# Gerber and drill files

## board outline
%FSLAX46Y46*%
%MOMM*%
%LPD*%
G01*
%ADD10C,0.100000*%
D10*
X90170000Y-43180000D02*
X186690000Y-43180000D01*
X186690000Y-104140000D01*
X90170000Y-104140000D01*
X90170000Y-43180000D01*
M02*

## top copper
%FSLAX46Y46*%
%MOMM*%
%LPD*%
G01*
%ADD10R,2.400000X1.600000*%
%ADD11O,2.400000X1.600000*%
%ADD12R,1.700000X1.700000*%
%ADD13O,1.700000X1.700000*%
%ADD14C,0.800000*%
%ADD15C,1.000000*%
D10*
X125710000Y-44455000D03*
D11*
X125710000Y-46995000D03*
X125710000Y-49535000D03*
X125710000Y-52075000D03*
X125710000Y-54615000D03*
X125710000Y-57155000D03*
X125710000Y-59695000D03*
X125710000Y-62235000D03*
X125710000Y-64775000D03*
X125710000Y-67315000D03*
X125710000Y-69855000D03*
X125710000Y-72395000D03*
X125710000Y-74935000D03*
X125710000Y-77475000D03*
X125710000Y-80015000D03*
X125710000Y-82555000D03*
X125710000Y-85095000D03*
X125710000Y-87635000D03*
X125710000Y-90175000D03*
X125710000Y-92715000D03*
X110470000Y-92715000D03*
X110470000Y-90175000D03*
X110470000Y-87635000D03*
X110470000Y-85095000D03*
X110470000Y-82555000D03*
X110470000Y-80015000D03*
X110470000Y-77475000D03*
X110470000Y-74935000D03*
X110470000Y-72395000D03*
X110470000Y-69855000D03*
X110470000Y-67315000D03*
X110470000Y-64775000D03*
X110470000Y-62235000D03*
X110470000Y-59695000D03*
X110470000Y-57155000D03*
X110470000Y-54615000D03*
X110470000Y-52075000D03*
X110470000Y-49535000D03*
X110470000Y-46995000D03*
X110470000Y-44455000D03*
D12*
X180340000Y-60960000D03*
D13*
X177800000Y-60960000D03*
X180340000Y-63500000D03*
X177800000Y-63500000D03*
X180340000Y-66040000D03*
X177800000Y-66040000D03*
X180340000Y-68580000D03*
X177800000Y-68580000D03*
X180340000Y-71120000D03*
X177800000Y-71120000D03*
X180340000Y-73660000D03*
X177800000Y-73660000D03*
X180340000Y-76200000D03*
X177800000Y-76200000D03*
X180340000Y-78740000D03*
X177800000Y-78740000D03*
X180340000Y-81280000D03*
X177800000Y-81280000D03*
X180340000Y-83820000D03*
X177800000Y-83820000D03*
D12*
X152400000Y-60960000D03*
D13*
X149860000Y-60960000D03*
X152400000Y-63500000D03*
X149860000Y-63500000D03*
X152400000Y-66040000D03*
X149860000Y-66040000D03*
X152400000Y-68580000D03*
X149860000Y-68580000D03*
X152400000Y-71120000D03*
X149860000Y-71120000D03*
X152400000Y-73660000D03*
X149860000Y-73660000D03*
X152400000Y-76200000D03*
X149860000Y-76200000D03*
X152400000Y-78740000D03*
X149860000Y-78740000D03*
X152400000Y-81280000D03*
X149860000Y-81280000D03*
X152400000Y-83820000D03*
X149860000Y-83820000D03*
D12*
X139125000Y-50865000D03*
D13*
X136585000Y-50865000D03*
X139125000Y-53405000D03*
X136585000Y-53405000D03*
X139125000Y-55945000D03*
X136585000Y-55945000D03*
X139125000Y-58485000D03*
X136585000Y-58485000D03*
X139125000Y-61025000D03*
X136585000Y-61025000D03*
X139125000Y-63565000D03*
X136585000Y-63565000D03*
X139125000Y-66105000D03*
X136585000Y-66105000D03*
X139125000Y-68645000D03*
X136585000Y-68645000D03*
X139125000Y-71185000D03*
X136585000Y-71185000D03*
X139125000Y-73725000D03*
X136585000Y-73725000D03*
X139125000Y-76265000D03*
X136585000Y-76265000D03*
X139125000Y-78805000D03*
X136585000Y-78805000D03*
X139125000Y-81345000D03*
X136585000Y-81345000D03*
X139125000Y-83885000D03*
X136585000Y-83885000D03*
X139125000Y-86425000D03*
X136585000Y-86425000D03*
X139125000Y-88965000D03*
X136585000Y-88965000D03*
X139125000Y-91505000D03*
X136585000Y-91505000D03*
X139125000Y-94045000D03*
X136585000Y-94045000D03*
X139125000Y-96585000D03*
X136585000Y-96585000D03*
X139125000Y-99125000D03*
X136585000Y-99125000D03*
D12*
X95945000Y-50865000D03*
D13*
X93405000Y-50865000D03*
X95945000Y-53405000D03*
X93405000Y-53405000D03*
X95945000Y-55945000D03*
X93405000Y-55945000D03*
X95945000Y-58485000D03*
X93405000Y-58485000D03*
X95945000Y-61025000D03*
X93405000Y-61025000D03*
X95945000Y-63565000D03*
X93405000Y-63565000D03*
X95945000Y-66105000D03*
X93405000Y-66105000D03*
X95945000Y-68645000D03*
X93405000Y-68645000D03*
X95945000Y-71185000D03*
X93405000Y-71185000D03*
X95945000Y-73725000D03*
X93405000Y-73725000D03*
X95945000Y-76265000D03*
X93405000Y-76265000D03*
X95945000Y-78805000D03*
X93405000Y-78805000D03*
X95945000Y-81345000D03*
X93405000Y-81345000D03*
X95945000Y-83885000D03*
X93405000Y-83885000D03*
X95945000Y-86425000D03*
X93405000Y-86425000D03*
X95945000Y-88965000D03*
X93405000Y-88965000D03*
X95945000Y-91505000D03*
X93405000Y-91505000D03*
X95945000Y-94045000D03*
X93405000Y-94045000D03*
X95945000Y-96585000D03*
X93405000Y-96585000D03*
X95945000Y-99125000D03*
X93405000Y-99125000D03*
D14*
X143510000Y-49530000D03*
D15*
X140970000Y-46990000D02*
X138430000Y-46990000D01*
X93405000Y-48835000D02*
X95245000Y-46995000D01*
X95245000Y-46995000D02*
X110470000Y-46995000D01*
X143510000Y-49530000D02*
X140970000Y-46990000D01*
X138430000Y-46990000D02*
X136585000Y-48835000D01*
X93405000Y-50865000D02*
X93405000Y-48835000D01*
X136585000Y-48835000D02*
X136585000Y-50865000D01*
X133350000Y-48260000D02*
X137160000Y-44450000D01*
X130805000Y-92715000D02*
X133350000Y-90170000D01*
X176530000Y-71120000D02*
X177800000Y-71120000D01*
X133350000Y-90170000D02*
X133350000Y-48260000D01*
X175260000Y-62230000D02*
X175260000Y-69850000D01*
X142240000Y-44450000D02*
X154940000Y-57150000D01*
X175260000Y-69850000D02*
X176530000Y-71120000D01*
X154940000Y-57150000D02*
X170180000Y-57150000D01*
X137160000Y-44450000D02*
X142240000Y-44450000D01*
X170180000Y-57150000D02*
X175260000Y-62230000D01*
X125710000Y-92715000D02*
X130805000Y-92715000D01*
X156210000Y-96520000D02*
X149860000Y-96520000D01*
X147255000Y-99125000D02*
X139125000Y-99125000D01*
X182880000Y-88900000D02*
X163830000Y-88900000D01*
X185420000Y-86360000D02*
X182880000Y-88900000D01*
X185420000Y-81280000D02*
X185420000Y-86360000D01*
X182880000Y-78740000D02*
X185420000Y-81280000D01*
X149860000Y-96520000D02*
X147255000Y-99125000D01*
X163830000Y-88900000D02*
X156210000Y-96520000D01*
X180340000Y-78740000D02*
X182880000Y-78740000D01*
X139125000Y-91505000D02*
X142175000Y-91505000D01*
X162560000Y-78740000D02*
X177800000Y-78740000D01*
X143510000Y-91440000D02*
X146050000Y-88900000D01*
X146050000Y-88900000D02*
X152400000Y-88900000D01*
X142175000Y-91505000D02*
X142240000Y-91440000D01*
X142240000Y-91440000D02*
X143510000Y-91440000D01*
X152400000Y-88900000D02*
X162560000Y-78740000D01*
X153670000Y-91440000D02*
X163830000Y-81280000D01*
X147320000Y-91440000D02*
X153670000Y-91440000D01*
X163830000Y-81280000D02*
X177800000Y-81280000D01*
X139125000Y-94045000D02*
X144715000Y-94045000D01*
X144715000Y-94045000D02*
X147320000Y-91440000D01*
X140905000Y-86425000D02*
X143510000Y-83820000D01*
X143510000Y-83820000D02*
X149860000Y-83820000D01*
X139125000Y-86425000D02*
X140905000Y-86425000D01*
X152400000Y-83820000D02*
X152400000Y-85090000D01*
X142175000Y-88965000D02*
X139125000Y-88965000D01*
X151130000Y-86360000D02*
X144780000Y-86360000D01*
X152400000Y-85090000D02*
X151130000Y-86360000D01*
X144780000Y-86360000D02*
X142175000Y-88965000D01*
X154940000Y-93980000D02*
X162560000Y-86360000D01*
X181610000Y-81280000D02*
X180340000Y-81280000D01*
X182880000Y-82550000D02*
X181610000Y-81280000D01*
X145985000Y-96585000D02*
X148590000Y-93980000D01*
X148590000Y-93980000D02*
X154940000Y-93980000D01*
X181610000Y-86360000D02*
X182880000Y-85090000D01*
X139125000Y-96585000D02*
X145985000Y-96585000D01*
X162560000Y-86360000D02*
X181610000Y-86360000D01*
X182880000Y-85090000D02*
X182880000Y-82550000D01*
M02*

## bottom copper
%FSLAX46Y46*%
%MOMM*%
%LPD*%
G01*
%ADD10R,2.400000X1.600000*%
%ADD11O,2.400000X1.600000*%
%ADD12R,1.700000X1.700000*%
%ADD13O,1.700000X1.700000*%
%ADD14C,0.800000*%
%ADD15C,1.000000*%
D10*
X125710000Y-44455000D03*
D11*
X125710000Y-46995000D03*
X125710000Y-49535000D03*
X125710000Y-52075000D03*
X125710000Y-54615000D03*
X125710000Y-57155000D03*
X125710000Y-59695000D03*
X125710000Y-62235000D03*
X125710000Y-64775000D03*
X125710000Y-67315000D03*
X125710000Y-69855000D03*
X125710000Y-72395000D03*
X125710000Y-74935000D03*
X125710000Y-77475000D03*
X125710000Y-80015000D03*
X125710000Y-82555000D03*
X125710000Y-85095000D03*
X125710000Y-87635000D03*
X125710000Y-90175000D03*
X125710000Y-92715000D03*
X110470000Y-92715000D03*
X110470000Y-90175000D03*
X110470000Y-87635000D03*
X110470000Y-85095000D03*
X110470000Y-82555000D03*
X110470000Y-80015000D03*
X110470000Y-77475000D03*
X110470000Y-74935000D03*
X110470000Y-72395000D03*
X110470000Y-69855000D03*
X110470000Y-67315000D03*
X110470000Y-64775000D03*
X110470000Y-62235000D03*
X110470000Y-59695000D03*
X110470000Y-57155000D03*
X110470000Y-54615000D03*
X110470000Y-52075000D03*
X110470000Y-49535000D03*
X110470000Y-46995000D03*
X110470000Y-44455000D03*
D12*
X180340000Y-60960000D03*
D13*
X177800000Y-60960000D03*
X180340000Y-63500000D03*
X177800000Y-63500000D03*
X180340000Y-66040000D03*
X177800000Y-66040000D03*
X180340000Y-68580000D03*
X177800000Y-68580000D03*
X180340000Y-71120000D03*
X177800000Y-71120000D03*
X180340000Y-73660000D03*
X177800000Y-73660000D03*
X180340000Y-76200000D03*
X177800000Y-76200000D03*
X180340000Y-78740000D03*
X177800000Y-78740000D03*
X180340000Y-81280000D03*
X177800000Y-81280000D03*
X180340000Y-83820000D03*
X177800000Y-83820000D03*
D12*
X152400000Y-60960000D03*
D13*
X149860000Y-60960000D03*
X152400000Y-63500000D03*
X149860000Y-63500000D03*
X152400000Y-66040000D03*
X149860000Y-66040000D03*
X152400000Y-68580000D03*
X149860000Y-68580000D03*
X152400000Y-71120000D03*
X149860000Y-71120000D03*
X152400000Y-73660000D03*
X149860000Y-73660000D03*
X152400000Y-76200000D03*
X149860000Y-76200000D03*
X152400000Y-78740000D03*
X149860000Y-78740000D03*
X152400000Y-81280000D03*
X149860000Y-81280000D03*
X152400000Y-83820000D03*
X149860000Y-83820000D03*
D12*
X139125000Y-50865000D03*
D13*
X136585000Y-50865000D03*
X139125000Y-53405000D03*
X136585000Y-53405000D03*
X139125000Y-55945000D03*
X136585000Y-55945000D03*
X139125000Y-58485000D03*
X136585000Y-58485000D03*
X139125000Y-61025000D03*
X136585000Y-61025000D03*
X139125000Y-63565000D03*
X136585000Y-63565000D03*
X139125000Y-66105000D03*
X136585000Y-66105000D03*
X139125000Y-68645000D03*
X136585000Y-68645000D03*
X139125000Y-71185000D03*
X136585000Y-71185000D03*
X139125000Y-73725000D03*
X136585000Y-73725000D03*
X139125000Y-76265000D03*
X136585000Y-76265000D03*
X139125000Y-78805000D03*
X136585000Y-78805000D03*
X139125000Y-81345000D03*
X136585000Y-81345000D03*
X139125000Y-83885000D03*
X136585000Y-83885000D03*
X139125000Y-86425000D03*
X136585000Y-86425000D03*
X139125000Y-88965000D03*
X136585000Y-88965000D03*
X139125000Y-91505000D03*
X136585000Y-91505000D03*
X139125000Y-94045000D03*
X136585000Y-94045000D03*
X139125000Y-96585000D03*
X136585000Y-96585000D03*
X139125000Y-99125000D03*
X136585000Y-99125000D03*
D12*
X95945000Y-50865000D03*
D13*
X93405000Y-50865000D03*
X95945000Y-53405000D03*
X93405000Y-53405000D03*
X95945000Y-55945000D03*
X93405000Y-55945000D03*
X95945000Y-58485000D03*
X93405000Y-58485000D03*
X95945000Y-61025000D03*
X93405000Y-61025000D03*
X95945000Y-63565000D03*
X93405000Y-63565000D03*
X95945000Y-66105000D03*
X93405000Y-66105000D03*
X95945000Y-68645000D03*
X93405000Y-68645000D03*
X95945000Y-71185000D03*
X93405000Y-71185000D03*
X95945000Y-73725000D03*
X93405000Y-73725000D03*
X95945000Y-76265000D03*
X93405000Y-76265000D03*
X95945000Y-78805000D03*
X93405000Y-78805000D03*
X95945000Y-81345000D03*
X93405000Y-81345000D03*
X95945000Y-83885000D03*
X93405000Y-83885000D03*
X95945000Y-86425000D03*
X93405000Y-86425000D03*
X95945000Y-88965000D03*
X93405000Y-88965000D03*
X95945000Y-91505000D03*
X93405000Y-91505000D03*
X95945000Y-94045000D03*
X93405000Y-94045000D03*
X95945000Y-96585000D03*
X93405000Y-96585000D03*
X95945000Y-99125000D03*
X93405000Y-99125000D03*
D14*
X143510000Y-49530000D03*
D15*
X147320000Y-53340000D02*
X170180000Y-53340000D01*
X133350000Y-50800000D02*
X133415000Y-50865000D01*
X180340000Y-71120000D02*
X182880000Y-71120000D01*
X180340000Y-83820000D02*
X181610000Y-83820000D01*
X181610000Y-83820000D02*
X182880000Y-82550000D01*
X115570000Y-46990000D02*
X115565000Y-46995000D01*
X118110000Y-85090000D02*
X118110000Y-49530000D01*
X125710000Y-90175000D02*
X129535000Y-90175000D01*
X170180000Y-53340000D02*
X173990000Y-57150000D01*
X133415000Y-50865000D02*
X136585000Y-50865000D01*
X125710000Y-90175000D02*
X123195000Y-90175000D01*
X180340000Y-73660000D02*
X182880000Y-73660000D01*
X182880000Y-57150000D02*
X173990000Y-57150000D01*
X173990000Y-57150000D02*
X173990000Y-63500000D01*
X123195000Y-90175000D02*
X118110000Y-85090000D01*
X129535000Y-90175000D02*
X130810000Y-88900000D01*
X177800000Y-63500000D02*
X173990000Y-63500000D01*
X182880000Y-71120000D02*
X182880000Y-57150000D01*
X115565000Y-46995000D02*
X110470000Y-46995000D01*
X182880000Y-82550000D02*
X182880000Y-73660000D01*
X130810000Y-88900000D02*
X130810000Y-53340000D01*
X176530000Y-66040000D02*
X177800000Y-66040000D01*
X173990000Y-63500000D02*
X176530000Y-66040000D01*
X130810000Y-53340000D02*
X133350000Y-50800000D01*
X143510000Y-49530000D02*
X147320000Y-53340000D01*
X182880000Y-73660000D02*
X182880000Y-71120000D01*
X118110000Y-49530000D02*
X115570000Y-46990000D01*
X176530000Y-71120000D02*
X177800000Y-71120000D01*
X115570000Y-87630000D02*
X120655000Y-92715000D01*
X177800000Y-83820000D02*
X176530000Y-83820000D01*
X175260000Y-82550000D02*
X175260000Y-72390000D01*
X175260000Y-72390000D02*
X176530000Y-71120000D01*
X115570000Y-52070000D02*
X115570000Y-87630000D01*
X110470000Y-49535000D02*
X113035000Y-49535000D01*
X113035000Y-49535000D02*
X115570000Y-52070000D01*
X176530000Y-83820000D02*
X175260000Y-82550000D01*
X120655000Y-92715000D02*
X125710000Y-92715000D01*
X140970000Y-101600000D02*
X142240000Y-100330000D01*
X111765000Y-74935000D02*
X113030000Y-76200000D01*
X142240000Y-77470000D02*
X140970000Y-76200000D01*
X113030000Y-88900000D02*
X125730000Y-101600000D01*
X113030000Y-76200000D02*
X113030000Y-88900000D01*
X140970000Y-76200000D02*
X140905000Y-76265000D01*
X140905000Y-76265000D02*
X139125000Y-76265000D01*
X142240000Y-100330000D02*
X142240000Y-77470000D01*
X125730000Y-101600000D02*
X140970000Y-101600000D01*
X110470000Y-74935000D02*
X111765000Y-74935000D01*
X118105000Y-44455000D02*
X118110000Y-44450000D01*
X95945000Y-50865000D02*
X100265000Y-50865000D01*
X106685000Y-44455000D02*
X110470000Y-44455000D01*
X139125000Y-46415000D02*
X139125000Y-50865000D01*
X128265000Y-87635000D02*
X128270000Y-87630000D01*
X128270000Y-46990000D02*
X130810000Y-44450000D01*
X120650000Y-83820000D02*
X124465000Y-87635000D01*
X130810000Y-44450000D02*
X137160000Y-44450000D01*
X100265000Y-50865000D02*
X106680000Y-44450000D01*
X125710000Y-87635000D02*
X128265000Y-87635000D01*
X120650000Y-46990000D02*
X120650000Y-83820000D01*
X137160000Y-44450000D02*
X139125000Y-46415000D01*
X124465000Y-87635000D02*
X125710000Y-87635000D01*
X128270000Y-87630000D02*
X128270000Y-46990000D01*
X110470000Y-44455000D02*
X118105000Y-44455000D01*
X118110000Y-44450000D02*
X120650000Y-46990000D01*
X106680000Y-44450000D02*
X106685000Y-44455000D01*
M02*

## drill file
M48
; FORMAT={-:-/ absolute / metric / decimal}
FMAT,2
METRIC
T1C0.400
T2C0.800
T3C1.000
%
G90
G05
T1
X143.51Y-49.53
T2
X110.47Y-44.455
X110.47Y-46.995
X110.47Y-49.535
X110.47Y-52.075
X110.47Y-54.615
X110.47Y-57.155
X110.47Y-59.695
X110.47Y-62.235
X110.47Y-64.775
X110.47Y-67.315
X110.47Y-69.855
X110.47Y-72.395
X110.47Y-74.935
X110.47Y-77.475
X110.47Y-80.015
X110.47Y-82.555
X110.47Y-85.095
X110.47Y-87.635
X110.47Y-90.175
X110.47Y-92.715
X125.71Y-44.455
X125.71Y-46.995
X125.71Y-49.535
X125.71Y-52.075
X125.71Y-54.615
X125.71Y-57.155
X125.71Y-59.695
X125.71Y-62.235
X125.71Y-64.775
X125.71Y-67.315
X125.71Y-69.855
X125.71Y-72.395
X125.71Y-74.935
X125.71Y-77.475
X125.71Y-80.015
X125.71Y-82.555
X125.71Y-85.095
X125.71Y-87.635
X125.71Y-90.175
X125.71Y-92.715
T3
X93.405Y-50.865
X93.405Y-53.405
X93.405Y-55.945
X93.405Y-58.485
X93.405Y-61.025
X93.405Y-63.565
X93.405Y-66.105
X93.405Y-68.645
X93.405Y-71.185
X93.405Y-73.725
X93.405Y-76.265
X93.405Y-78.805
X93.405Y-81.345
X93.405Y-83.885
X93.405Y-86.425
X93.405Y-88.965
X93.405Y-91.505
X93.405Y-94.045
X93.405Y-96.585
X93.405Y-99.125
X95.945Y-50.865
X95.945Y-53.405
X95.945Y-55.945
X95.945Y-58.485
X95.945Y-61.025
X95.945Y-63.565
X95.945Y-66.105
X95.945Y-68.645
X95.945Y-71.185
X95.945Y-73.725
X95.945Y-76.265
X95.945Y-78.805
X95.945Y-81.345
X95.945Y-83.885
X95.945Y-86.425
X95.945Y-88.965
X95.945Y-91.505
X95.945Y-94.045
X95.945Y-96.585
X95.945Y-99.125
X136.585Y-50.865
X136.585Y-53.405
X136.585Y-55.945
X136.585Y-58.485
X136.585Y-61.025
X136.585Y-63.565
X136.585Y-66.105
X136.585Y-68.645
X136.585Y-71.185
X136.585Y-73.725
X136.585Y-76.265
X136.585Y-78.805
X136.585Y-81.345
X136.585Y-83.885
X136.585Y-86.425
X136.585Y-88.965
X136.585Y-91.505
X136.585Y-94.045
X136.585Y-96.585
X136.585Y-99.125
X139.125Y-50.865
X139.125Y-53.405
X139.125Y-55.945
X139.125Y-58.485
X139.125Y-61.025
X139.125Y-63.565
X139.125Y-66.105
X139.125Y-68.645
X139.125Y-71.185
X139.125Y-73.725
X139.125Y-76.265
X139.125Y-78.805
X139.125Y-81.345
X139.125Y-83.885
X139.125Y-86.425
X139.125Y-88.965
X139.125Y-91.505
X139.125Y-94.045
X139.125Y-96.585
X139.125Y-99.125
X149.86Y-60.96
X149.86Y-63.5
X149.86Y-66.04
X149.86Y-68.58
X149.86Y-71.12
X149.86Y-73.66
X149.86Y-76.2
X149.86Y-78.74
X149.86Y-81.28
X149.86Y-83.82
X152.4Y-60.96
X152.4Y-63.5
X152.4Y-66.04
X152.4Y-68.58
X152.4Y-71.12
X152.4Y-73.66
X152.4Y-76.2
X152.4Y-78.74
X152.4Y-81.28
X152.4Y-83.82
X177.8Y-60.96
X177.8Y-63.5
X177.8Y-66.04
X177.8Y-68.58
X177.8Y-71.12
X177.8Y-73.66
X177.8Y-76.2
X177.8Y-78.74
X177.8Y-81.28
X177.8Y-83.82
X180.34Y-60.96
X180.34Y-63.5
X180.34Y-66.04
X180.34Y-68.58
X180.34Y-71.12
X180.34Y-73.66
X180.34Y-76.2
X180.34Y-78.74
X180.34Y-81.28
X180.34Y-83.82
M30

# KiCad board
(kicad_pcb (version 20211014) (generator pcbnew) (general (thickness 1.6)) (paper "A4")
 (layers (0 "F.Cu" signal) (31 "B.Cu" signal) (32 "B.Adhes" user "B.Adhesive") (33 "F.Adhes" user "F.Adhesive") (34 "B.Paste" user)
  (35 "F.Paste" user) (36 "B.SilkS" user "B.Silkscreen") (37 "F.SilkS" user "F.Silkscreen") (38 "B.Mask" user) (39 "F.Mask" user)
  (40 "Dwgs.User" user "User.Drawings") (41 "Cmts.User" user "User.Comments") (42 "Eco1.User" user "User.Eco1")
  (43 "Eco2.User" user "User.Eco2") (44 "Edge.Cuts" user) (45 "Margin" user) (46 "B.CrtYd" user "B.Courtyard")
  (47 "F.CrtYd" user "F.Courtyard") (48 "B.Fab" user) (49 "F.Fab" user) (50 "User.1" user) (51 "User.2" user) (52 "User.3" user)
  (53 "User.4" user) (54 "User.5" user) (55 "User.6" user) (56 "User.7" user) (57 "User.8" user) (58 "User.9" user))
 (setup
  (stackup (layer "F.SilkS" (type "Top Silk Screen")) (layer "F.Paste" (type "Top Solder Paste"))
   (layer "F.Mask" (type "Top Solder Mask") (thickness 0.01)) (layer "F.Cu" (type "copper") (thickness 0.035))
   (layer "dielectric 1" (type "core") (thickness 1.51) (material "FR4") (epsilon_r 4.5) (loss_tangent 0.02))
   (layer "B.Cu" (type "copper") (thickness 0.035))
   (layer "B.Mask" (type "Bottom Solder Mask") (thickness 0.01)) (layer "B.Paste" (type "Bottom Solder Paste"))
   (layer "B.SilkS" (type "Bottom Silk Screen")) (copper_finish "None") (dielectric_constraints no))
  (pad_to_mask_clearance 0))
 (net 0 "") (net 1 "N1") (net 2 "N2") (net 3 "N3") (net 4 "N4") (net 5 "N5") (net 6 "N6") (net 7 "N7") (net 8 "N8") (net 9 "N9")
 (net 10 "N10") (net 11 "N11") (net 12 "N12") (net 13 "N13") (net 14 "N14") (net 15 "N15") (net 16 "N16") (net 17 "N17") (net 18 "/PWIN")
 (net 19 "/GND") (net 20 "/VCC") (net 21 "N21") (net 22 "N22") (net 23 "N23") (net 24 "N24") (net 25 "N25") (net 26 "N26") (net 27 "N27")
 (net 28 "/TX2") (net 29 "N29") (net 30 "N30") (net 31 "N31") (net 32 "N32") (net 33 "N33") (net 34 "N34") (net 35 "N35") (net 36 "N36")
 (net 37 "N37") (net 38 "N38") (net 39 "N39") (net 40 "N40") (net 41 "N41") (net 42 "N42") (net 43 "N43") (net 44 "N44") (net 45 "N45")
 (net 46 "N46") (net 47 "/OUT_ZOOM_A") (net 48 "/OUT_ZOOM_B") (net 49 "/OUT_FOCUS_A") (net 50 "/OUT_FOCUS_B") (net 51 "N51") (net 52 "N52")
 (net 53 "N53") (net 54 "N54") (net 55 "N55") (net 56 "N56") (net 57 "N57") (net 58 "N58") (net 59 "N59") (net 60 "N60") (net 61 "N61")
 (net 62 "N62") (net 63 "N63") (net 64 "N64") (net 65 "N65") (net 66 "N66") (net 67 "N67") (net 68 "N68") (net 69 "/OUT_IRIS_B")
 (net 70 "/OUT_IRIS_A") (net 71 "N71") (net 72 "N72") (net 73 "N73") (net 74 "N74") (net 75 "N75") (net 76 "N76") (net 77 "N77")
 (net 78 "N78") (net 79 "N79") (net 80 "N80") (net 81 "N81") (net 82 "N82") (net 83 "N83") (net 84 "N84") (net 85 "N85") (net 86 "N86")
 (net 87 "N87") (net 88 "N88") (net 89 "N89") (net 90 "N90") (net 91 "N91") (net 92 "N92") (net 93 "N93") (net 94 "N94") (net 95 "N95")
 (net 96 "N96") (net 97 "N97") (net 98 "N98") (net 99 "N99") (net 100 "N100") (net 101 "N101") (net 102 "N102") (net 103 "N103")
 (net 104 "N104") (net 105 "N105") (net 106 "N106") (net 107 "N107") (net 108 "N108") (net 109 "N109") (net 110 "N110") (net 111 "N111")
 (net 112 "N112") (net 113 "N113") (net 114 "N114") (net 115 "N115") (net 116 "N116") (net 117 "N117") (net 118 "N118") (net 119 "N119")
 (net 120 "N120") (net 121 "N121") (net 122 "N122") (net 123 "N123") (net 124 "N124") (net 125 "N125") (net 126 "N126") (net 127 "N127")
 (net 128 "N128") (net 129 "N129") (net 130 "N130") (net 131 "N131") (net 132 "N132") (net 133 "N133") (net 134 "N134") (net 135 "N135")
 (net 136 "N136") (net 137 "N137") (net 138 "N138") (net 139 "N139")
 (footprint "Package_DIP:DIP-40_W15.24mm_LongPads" (layer "B.Cu") (at 125.71 44.455 180)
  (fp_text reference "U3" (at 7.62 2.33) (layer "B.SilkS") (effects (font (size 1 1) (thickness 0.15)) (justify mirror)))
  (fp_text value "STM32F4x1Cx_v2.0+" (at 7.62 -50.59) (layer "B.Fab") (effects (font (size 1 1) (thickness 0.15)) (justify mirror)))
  (pad "1" thru_hole rect locked (at 0 0 180) (size 2.4 1.6) (drill 0.8) (layers *.Cu *.Mask) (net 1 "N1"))
  (pad "2" thru_hole oval locked (at 0 -2.54 180) (size 2.4 1.6) (drill 0.8) (layers *.Cu *.Mask) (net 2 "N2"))
  (pad "3" thru_hole oval locked (at 0 -5.08 180) (size 2.4 1.6) (drill 0.8) (layers *.Cu *.Mask) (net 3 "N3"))
  (pad "4" thru_hole oval locked (at 0 -7.62 180) (size 2.4 1.6) (drill 0.8) (layers *.Cu *.Mask) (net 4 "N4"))
  (pad "5" thru_hole oval locked (at 0 -10.16 180) (size 2.4 1.6) (drill 0.8) (layers *.Cu *.Mask) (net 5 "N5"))
  (pad "6" thru_hole oval locked (at 0 -12.7 180) (size 2.4 1.6) (drill 0.8) (layers *.Cu *.Mask) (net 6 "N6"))
  (pad "7" thru_hole oval locked (at 0 -15.24 180) (size 2.4 1.6) (drill 0.8) (layers *.Cu *.Mask) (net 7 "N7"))
  (pad "8" thru_hole oval locked (at 0 -17.78 180) (size 2.4 1.6) (drill 0.8) (layers *.Cu *.Mask) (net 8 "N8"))
  (pad "9" thru_hole oval locked (at 0 -20.32 180) (size 2.4 1.6) (drill 0.8) (layers *.Cu *.Mask) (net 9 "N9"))
  (pad "10" thru_hole oval locked (at 0 -22.86 180) (size 2.4 1.6) (drill 0.8) (layers *.Cu *.Mask) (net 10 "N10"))
  (pad "11" thru_hole oval locked (at 0 -25.4 180) (size 2.4 1.6) (drill 0.8) (layers *.Cu *.Mask) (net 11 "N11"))
  (pad "12" thru_hole oval locked (at 0 -27.94 180) (size 2.4 1.6) (drill 0.8) (layers *.Cu *.Mask) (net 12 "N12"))
  (pad "13" thru_hole oval locked (at 0 -30.48 180) (size 2.4 1.6) (drill 0.8) (layers *.Cu *.Mask) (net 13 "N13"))
  (pad "14" thru_hole oval locked (at 0 -33.02 180) (size 2.4 1.6) (drill 0.8) (layers *.Cu *.Mask) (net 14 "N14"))
  (pad "15" thru_hole oval locked (at 0 -35.56 180) (size 2.4 1.6) (drill 0.8) (layers *.Cu *.Mask) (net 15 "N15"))
  (pad "16" thru_hole oval locked (at 0 -38.1 180) (size 2.4 1.6) (drill 0.8) (layers *.Cu *.Mask) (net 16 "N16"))
  (pad "17" thru_hole oval locked (at 0 -40.64 180) (size 2.4 1.6) (drill 0.8) (layers *.Cu *.Mask) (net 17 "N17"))
  (pad "18" thru_hole oval locked (at 0 -43.18 180) (size 2.4 1.6) (drill 0.8) (layers *.Cu *.Mask) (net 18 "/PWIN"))
  (pad "19" thru_hole oval locked (at 0 -45.72 180) (size 2.4 1.6) (drill 0.8) (layers *.Cu *.Mask) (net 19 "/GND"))
  (pad "20" thru_hole oval locked (at 0 -48.26 180) (size 2.4 1.6) (drill 0.8) (layers *.Cu *.Mask) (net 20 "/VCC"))
  (pad "21" thru_hole oval locked (at 15.24 -48.26 180) (size 2.4 1.6) (drill 0.8) (layers *.Cu *.Mask) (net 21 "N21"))
  (pad "22" thru_hole oval locked (at 15.24 -45.72 180) (size 2.4 1.6) (drill 0.8) (layers *.Cu *.Mask) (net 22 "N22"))
  (pad "23" thru_hole oval locked (at 15.24 -43.18 180) (size 2.4 1.6) (drill 0.8) (layers *.Cu *.Mask) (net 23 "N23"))
  (pad "24" thru_hole oval locked (at 15.24 -40.64 180) (size 2.4 1.6) (drill 0.8) (layers *.Cu *.Mask) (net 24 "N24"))
  (pad "25" thru_hole oval locked (at 15.24 -38.1 180) (size 2.4 1.6) (drill 0.8) (layers *.Cu *.Mask) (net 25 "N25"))
  (pad "26" thru_hole oval locked (at 15.24 -35.56 180) (size 2.4 1.6) (drill 0.8) (layers *.Cu *.Mask) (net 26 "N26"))
  (pad "27" thru_hole oval locked (at 15.24 -33.02 180) (size 2.4 1.6) (drill 0.8) (layers *.Cu *.Mask) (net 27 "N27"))
  (pad "28" thru_hole oval locked (at 15.24 -30.48 180) (size 2.4 1.6) (drill 0.8) (layers *.Cu *.Mask) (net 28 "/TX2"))
  (pad "29" thru_hole oval locked (at 15.24 -27.94 180) (size 2.4 1.6) (drill 0.8) (layers *.Cu *.Mask) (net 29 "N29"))
  (pad "30" thru_hole oval locked (at 15.24 -25.4 180) (size 2.4 1.6) (drill 0.8) (layers *.Cu *.Mask) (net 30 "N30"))
  (pad "31" thru_hole oval locked (at 15.24 -22.86 180) (size 2.4 1.6) (drill 0.8) (layers *.Cu *.Mask) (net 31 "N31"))
  (pad "32" thru_hole oval locked (at 15.24 -20.32 180) (size 2.4 1.6) (drill 0.8) (layers *.Cu *.Mask) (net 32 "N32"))
  (pad "33" thru_hole oval locked (at 15.24 -17.78 180) (size 2.4 1.6) (drill 0.8) (layers *.Cu *.Mask) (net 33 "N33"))
  (pad "34" thru_hole oval locked (at 15.24 -15.24 180) (size 2.4 1.6) (drill 0.8) (layers *.Cu *.Mask) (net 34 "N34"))
  (pad "35" thru_hole oval locked (at 15.24 -12.7 180) (size 2.4 1.6) (drill 0.8) (layers *.Cu *.Mask) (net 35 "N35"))
  (pad "36" thru_hole oval locked (at 15.24 -10.16 180) (size 2.4 1.6) (drill 0.8) (layers *.Cu *.Mask) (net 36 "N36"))
  (pad "37" thru_hole oval locked (at 15.24 -7.62 180) (size 2.4 1.6) (drill 0.8) (layers *.Cu *.Mask) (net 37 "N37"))
  (pad "38" thru_hole oval locked (at 15.24 -5.08 180) (size 2.4 1.6) (drill 0.8) (layers *.Cu *.Mask) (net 20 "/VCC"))
  (pad "39" thru_hole oval locked (at 15.24 -2.54 180) (size 2.4 1.6) (drill 0.8) (layers *.Cu *.Mask) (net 19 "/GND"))
  (pad "40" thru_hole oval locked (at 15.24 0 180) (size 2.4 1.6) (drill 0.8) (layers *.Cu *.Mask) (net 18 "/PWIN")))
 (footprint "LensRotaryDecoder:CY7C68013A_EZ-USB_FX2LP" (layer "B.Cu") (at 168.37 72.385 180)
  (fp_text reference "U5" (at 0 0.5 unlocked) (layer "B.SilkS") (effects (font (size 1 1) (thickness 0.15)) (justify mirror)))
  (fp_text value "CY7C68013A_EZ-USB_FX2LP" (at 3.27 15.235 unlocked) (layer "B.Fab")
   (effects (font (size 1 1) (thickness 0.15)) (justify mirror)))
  (pad "1" thru_hole rect (at -11.97 11.425 180) (size 1.7 1.7) (drill 1) (layers *.Cu *.Mask) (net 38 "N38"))
  (pad "2" thru_hole oval (at -9.43 11.425 180) (size 1.7 1.7) (drill 1) (layers *.Cu *.Mask) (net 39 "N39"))
  (pad "3" thru_hole oval (at -11.97 8.885 180) (size 1.7 1.7) (drill 1) (layers *.Cu *.Mask) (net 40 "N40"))
  (pad "4" thru_hole oval (at -9.43 8.885 180) (size 1.7 1.7) (drill 1) (layers *.Cu *.Mask) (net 19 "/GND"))
  (pad "5" thru_hole oval (at -11.97 6.345 180) (size 1.7 1.7) (drill 1) (layers *.Cu *.Mask) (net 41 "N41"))
  (pad "6" thru_hole oval (at -9.43 6.345 180) (size 1.7 1.7) (drill 1) (layers *.Cu *.Mask) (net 19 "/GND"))
  (pad "7" thru_hole oval (at -11.97 3.805 180) (size 1.7 1.7) (drill 1) (layers *.Cu *.Mask) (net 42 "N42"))
  (pad "8" thru_hole oval (at -9.43 3.805 180) (size 1.7 1.7) (drill 1) (layers *.Cu *.Mask) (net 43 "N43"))
  (pad "9" thru_hole oval (at -11.97 1.265 180) (size 1.7 1.7) (drill 1) (layers *.Cu *.Mask) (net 19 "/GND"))
  (pad "10" thru_hole oval (at -9.43 1.265 180) (size 1.7 1.7) (drill 1) (layers *.Cu *.Mask) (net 20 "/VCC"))
  (pad "11" thru_hole oval (at -11.97 -1.275 180) (size 1.7 1.7) (drill 1) (layers *.Cu *.Mask) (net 19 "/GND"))
  (pad "12" thru_hole oval (at -9.43 -1.275 180) (size 1.7 1.7) (drill 1) (layers *.Cu *.Mask) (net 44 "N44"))
  (pad "13" thru_hole oval (at -11.97 -3.815 180) (size 1.7 1.7) (drill 1) (layers *.Cu *.Mask) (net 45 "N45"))
  (pad "14" thru_hole oval (at -9.43 -3.815 180) (size 1.7 1.7) (drill 1) (layers *.Cu *.Mask) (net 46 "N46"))
  (pad "15" thru_hole oval (at -11.97 -6.355 180) (size 1.7 1.7) (drill 1) (layers *.Cu *.Mask) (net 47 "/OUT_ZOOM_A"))
  (pad "16" thru_hole oval (at -9.43 -6.355 180) (size 1.7 1.7) (drill 1) (layers *.Cu *.Mask) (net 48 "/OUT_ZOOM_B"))
  (pad "17" thru_hole oval (at -11.97 -8.895 180) (size 1.7 1.7) (drill 1) (layers *.Cu *.Mask) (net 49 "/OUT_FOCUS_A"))
  (pad "18" thru_hole oval (at -9.43 -8.895 180) (size 1.7 1.7) (drill 1) (layers *.Cu *.Mask) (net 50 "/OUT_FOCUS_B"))
  (pad "19" thru_hole oval (at -11.97 -11.435 180) (size 1.7 1.7) (drill 1) (layers *.Cu *.Mask) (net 19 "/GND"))
  (pad "20" thru_hole oval (at -9.43 -11.435 180) (size 1.7 1.7) (drill 1) (layers *.Cu *.Mask) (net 20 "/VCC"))
  (pad "21" thru_hole rect (at 15.97 11.425 180) (size 1.7 1.7) (drill 1) (layers *.Cu *.Mask) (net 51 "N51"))
  (pad "22" thru_hole oval (at 18.51 11.425 180) (size 1.7 1.7) (drill 1) (layers *.Cu *.Mask) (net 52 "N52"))
  (pad "23" thru_hole oval (at 15.97 8.885 180) (size 1.7 1.7) (drill 1) (layers *.Cu *.Mask) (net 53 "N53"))
  (pad "24" thru_hole oval (at 18.51 8.885 180) (size 1.7 1.7) (drill 1) (layers *.Cu *.Mask) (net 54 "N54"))
  (pad "25" thru_hole oval (at 15.97 6.345 180) (size 1.7 1.7) (drill 1) (layers *.Cu *.Mask) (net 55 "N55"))
  (pad "26" thru_hole oval (at 18.51 6.345 180) (size 1.7 1.7) (drill 1) (layers *.Cu *.Mask) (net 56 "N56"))
  (pad "27" thru_hole oval (at 15.97 3.805 180) (size 1.7 1.7) (drill 1) (layers *.Cu *.Mask) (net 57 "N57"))
  (pad "28" thru_hole oval (at 18.51 3.805 180) (size 1.7 1.7) (drill 1) (layers *.Cu *.Mask) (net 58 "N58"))
  (pad "29" thru_hole oval (at 15.97 1.265 180) (size 1.7 1.7) (drill 1) (layers *.Cu *.Mask) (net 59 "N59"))
  (pad "30" thru_hole oval (at 18.51 1.265 180) (size 1.7 1.7) (drill 1) (layers *.Cu *.Mask) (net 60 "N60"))
  (pad "31" thru_hole oval (at 15.97 -1.275 180) (size 1.7 1.7) (drill 1) (layers *.Cu *.Mask) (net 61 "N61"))
  (pad "32" thru_hole oval (at 18.51 -1.275 180) (size 1.7 1.7) (drill 1) (layers *.Cu *.Mask) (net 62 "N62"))
  (pad "33" thru_hole oval (at 15.97 -3.815 180) (size 1.7 1.7) (drill 1) (layers *.Cu *.Mask) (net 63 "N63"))
  (pad "34" thru_hole oval (at 18.51 -3.815 180) (size 1.7 1.7) (drill 1) (layers *.Cu *.Mask) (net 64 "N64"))
  (pad "35" thru_hole oval (at 15.97 -6.355 180) (size 1.7 1.7) (drill 1) (layers *.Cu *.Mask) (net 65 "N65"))
  (pad "36" thru_hole oval (at 18.51 -6.355 180) (size 1.7 1.7) (drill 1) (layers *.Cu *.Mask) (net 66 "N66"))
  (pad "37" thru_hole oval (at 15.97 -8.895 180) (size 1.7 1.7) (drill 1) (layers *.Cu *.Mask) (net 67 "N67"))
  (pad "38" thru_hole oval (at 18.51 -8.895 180) (size 1.7 1.7) (drill 1) (layers *.Cu *.Mask) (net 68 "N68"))
  (pad "39" thru_hole oval (at 15.97 -11.435 180) (size 1.7 1.7) (drill 1) (layers *.Cu *.Mask) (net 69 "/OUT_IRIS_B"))
  (pad "40" thru_hole oval (at 18.51 -11.435 180) (size 1.7 1.7) (drill 1) (layers *.Cu *.Mask) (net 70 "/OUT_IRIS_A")))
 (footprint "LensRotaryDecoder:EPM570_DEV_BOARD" (layer "B.Cu") (at 116.265 76.265 180)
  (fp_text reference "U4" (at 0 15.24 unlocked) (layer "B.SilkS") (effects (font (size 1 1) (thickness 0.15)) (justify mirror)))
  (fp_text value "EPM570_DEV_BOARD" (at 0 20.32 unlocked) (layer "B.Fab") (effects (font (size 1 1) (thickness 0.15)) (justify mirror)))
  (pad "1" thru_hole rect (at -22.86 25.4 180) (size 1.7 1.7) (drill 1) (layers *.Cu *.Mask) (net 18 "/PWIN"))
  (pad "2" thru_hole oval (at -20.32 25.4 180) (size 1.7 1.7) (drill 1) (layers *.Cu *.Mask) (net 19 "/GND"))
  (pad "3" thru_hole oval (at -22.86 22.86 180) (size 1.7 1.7) (drill 1) (layers *.Cu *.Mask) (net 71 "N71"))
  (pad "4" thru_hole oval (at -20.32 22.86 180) (size 1.7 1.7) (drill 1) (layers *.Cu *.Mask) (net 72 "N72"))
  (pad "5" thru_hole oval (at -22.86 20.32 180) (size 1.7 1.7) (drill 1) (layers *.Cu *.Mask) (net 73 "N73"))
  (pad "6" thru_hole oval (at -20.32 20.32 180) (size 1.7 1.7) (drill 1) (layers *.Cu *.Mask) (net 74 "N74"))
  (pad "7" thru_hole oval (at -22.86 17.78 180) (size 1.7 1.7) (drill 1) (layers *.Cu *.Mask) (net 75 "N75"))
  (pad "8" thru_hole oval (at -20.32 17.78 180) (size 1.7 1.7) (drill 1) (layers *.Cu *.Mask) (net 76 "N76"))
  (pad "9" thru_hole oval (at -22.86 15.24 180) (size 1.7 1.7) (drill 1) (layers *.Cu *.Mask) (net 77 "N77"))
  (pad "10" thru_hole oval (at -20.32 15.24 180) (size 1.7 1.7) (drill 1) (layers *.Cu *.Mask) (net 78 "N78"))
  (pad "11" thru_hole oval (at -22.86 12.7 180) (size 1.7 1.7) (drill 1) (layers *.Cu *.Mask) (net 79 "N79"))
  (pad "12" thru_hole oval (at -20.32 12.7 180) (size 1.7 1.7) (drill 1) (layers *.Cu *.Mask) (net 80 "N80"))
  (pad "13" thru_hole oval (at -22.86 10.16 180) (size 1.7 1.7) (drill 1) (layers *.Cu *.Mask) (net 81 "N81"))
  (pad "14" thru_hole oval (at -20.32 10.16 180) (size 1.7 1.7) (drill 1) (layers *.Cu *.Mask) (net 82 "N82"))
  (pad "15" thru_hole oval (at -22.86 7.62 180) (size 1.7 1.7) (drill 1) (layers *.Cu *.Mask) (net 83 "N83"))
  (pad "16" thru_hole oval (at -20.32 7.62 180) (size 1.7 1.7) (drill 1) (layers *.Cu *.Mask) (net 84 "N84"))
  (pad "17" thru_hole oval (at -22.86 5.08 180) (size 1.7 1.7) (drill 1) (layers *.Cu *.Mask) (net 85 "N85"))
  (pad "18" thru_hole oval (at -20.32 5.08 180) (size 1.7 1.7) (drill 1) (layers *.Cu *.Mask) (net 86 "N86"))
  (pad "19" thru_hole oval (at -22.86 2.54 180) (size 1.7 1.7) (drill 1) (layers *.Cu *.Mask) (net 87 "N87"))
  (pad "20" thru_hole oval (at -20.32 2.54 180) (size 1.7 1.7) (drill 1) (layers *.Cu *.Mask) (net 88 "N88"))
  (pad "21" thru_hole oval (at -22.86 0 180) (size 1.7 1.7) (drill 1) (layers *.Cu *.Mask) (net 28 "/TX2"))
  (pad "22" thru_hole oval (at -20.32 0 180) (size 1.7 1.7) (drill 1) (layers *.Cu *.Mask) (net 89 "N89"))
  (pad "23" thru_hole oval (at -22.86 -2.54 180) (size 1.7 1.7) (drill 1) (layers *.Cu *.Mask) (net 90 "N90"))
  (pad "24" thru_hole oval (at -20.32 -2.54 180) (size 1.7 1.7) (drill 1) (layers *.Cu *.Mask) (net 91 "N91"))
  (pad "25" thru_hole oval (at -22.86 -5.08 180) (size 1.7 1.7) (drill 1) (layers *.Cu *.Mask) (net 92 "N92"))
  (pad "26" thru_hole oval (at -20.32 -5.08 180) (size 1.7 1.7) (drill 1) (layers *.Cu *.Mask) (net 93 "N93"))
  (pad "27" thru_hole oval (at -22.86 -7.62 180) (size 1.7 1.7) (drill 1) (layers *.Cu *.Mask) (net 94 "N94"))
  (pad "28" thru_hole oval (at -20.32 -7.62 180) (size 1.7 1.7) (drill 1) (layers *.Cu *.Mask) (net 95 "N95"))
  (pad "29" thru_hole oval (at -22.86 -10.16 180) (size 1.7 1.7) (drill 1) (layers *.Cu *.Mask) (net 70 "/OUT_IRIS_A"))
  (pad "30" thru_hole oval (at -20.32 -10.16 180) (size 1.7 1.7) (drill 1) (layers *.Cu *.Mask) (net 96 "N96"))
  (pad "31" thru_hole oval (at -22.86 -12.7 180) (size 1.7 1.7) (drill 1) (layers *.Cu *.Mask) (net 69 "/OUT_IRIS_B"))
  (pad "32" thru_hole oval (at -20.32 -12.7 180) (size 1.7 1.7) (drill 1) (layers *.Cu *.Mask) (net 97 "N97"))
  (pad "33" thru_hole oval (at -22.86 -15.24 180) (size 1.7 1.7) (drill 1) (layers *.Cu *.Mask) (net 48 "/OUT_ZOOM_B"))
  (pad "34" thru_hole oval (at -20.32 -15.24 180) (size 1.7 1.7) (drill 1) (layers *.Cu *.Mask) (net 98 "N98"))
  (pad "35" thru_hole oval (at -22.86 -17.78 180) (size 1.7 1.7) (drill 1) (layers *.Cu *.Mask) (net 50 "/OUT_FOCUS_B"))
  (pad "36" thru_hole oval (at -20.32 -17.78 180) (size 1.7 1.7) (drill 1) (layers *.Cu *.Mask) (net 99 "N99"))
  (pad "37" thru_hole oval (at -22.86 -20.32 180) (size 1.7 1.7) (drill 1) (layers *.Cu *.Mask) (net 49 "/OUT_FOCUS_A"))
  (pad "38" thru_hole oval (at -20.32 -20.32 180) (size 1.7 1.7) (drill 1) (layers *.Cu *.Mask) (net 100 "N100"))
  (pad "39" thru_hole oval (at -22.86 -22.86 180) (size 1.7 1.7) (drill 1) (layers *.Cu *.Mask) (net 47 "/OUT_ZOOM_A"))
  (pad "40" thru_hole oval (at -20.32 -22.86 180) (size 1.7 1.7) (drill 1) (layers *.Cu *.Mask) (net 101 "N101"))
  (pad "41" thru_hole rect (at 20.32 25.4 180) (size 1.7 1.7) (drill 1) (layers *.Cu *.Mask) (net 18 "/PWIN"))
  (pad "42" thru_hole oval (at 22.86 25.4 180) (size 1.7 1.7) (drill 1) (layers *.Cu *.Mask) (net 19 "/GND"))
  (pad "43" thru_hole oval (at 20.32 22.86 180) (size 1.7 1.7) (drill 1) (layers *.Cu *.Mask) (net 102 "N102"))
  (pad "44" thru_hole oval (at 22.86 22.86 180) (size 1.7 1.7) (drill 1) (layers *.Cu *.Mask) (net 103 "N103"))
  (pad "45" thru_hole oval (at 20.32 20.32 180) (size 1.7 1.7) (drill 1) (layers *.Cu *.Mask) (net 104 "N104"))
  (pad "46" thru_hole oval (at 22.86 20.32 180) (size 1.7 1.7) (drill 1) (layers *.Cu *.Mask) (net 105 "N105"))
  (pad "47" thru_hole oval (at 20.32 17.78 180) (size 1.7 1.7) (drill 1) (layers *.Cu *.Mask) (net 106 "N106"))
  (pad "48" thru_hole oval (at 22.86 17.78 180) (size 1.7 1.7) (drill 1) (layers *.Cu *.Mask) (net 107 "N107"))
  (pad "49" thru_hole oval (at 20.32 15.24 180) (size 1.7 1.7) (drill 1) (layers *.Cu *.Mask) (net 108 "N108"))
  (pad "50" thru_hole oval (at 22.86 15.24 180) (size 1.7 1.7) (drill 1) (layers *.Cu *.Mask) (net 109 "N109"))
  (pad "51" thru_hole oval (at 20.32 12.7 180) (size 1.7 1.7) (drill 1) (layers *.Cu *.Mask) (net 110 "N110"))
  (pad "52" thru_hole oval (at 22.86 12.7 180) (size 1.7 1.7) (drill 1) (layers *.Cu *.Mask) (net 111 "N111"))
  (pad "53" thru_hole oval (at 20.32 10.16 180) (size 1.7 1.7) (drill 1) (layers *.Cu *.Mask) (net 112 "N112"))
  (pad "54" thru_hole oval (at 22.86 10.16 180) (size 1.7 1.7) (drill 1) (layers *.Cu *.Mask) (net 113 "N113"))
  (pad "55" thru_hole oval (at 20.32 7.62 180) (size 1.7 1.7) (drill 1) (layers *.Cu *.Mask) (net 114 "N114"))
  (pad "56" thru_hole oval (at 22.86 7.62 180) (size 1.7 1.7) (drill 1) (layers *.Cu *.Mask) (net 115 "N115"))
  (pad "57" thru_hole oval (at 20.32 5.08 180) (size 1.7 1.7) (drill 1) (layers *.Cu *.Mask) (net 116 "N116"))
  (pad "58" thru_hole oval (at 22.86 5.08 180) (size 1.7 1.7) (drill 1) (layers *.Cu *.Mask) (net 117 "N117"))
  (pad "59" thru_hole oval (at 20.32 2.54 180) (size 1.7 1.7) (drill 1) (layers *.Cu *.Mask) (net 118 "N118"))
  (pad "60" thru_hole oval (at 22.86 2.54 180) (size 1.7 1.7) (drill 1) (layers *.Cu *.Mask) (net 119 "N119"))
  (pad "61" thru_hole oval (at 20.32 0 180) (size 1.7 1.7) (drill 1) (layers *.Cu *.Mask) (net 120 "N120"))
  (pad "62" thru_hole oval (at 22.86 0 180) (size 1.7 1.7) (drill 1) (layers *.Cu *.Mask) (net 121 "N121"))
  (pad "63" thru_hole oval (at 20.32 -2.54 180) (size 1.7 1.7) (drill 1) (layers *.Cu *.Mask) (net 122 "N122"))
  (pad "64" thru_hole oval (at 22.86 -2.54 180) (size 1.7 1.7) (drill 1) (layers *.Cu *.Mask) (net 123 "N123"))
  (pad "65" thru_hole oval (at 20.32 -5.08 180) (size 1.7 1.7) (drill 1) (layers *.Cu *.Mask) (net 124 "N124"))
  (pad "66" thru_hole oval (at 22.86 -5.08 180) (size 1.7 1.7) (drill 1) (layers *.Cu *.Mask) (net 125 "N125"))
  (pad "67" thru_hole oval (at 20.32 -7.62 180) (size 1.7 1.7) (drill 1) (layers *.Cu *.Mask) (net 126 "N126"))
  (pad "68" thru_hole oval (at 22.86 -7.62 180) (size 1.7 1.7) (drill 1) (layers *.Cu *.Mask) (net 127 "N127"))
  (pad "69" thru_hole oval (at 20.32 -10.16 180) (size 1.7 1.7) (drill 1) (layers *.Cu *.Mask) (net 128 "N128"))
  (pad "70" thru_hole oval (at 22.86 -10.16 180) (size 1.7 1.7) (drill 1) (layers *.Cu *.Mask) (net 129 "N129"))
  (pad "71" thru_hole oval (at 20.32 -12.7 180) (size 1.7 1.7) (drill 1) (layers *.Cu *.Mask) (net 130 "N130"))
  (pad "72" thru_hole oval (at 22.86 -12.7 180) (size 1.7 1.7) (drill 1) (layers *.Cu *.Mask) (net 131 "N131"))
  (pad "73" thru_hole oval (at 20.32 -15.24 180) (size 1.7 1.7) (drill 1) (layers *.Cu *.Mask) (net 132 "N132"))
  (pad "74" thru_hole oval (at 22.86 -15.24 180) (size 1.7 1.7) (drill 1) (layers *.Cu *.Mask) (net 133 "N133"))
  (pad "75" thru_hole oval (at 20.32 -17.78 180) (size 1.7 1.7) (drill 1) (layers *.Cu *.Mask) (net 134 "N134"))
  (pad "76" thru_hole oval (at 22.86 -17.78 180) (size 1.7 1.7) (drill 1) (layers *.Cu *.Mask) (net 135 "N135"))
  (pad "77" thru_hole oval (at 20.32 -20.32 180) (size 1.7 1.7) (drill 1) (layers *.Cu *.Mask) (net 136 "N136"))
  (pad "78" thru_hole oval (at 22.86 -20.32 180) (size 1.7 1.7) (drill 1) (layers *.Cu *.Mask) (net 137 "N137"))
  (pad "79" thru_hole oval (at 20.32 -22.86 180) (size 1.7 1.7) (drill 1) (layers *.Cu *.Mask) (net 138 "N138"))
  (pad "80" thru_hole oval (at 22.86 -22.86 180) (size 1.7 1.7) (drill 1) (layers *.Cu *.Mask) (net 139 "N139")))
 (gr_rect (start 90.17 43.18) (end 186.69 104.14) (layer "Edge.Cuts") (width 0.1) (fill none))
 (segment (start 140.97 46.99) (end 138.43 46.99) (width 1) (layer "F.Cu") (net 19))
 (segment (start 93.405 48.835) (end 95.245 46.995) (width 1) (layer "F.Cu") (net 19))
 (segment (start 95.245 46.995) (end 110.47 46.995) (width 1) (layer "F.Cu") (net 19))
 (segment (start 143.51 49.53) (end 140.97 46.99) (width 1) (layer "F.Cu") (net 19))
 (segment (start 138.43 46.99) (end 136.585 48.835) (width 1) (layer "F.Cu") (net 19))
 (segment (start 93.405 50.865) (end 93.405 48.835) (width 1) (layer "F.Cu") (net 19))
 (segment (start 136.585 48.835) (end 136.585 50.865) (width 1) (layer "F.Cu") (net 19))
 (via (at 143.51 49.53) (size 0.8) (drill 0.4) (layers "F.Cu" "B.Cu") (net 19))
 (segment (start 147.32 53.34) (end 170.18 53.34) (width 1) (layer "B.Cu") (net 19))
 (segment (start 133.35 50.8) (end 133.415 50.865) (width 1) (layer "B.Cu") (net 19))
 (segment (start 180.34 71.12) (end 182.88 71.12) (width 1) (layer "B.Cu") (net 19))
 (segment (start 180.34 83.82) (end 181.61 83.82) (width 1) (layer "B.Cu") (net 19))
 (segment (start 181.61 83.82) (end 182.88 82.55) (width 1) (layer "B.Cu") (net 19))
 (segment (start 115.57 46.99) (end 115.565 46.995) (width 1) (layer "B.Cu") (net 19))
 (segment (start 118.11 85.09) (end 118.11 49.53) (width 1) (layer "B.Cu") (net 19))
 (segment (start 125.71 90.175) (end 129.535 90.175) (width 1) (layer "B.Cu") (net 19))
 (segment (start 170.18 53.34) (end 173.99 57.15) (width 1) (layer "B.Cu") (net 19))
 (segment (start 133.415 50.865) (end 136.585 50.865) (width 1) (layer "B.Cu") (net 19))
 (segment (start 125.71 90.175) (end 123.195 90.175) (width 1) (layer "B.Cu") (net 19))
 (segment (start 180.34 73.66) (end 182.88 73.66) (width 1) (layer "B.Cu") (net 19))
 (segment (start 182.88 57.15) (end 173.99 57.15) (width 1) (layer "B.Cu") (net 19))
 (segment (start 173.99 57.15) (end 173.99 63.5) (width 1) (layer "B.Cu") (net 19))
 (segment (start 123.195 90.175) (end 118.11 85.09) (width 1) (layer "B.Cu") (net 19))
 (segment (start 129.535 90.175) (end 130.81 88.9) (width 1) (layer "B.Cu") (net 19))
 (segment (start 177.8 63.5) (end 173.99 63.5) (width 1) (layer "B.Cu") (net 19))
 (segment (start 182.88 71.12) (end 182.88 57.15) (width 1) (layer "B.Cu") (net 19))
 (segment (start 115.565 46.995) (end 110.47 46.995) (width 1) (layer "B.Cu") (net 19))
 (segment (start 182.88 82.55) (end 182.88 73.66) (width 1) (layer "B.Cu") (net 19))
 (segment (start 130.81 88.9) (end 130.81 53.34) (width 1) (layer "B.Cu") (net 19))
 (segment (start 176.53 66.04) (end 177.8 66.04) (width 1) (layer "B.Cu") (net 19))
 (segment (start 173.99 63.5) (end 176.53 66.04) (width 1) (layer "B.Cu") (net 19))
 (segment (start 130.81 53.34) (end 133.35 50.8) (width 1) (layer "B.Cu") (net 19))
 (segment (start 143.51 49.53) (end 147.32 53.34) (width 1) (layer "B.Cu") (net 19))
 (segment (start 182.88 73.66) (end 182.88 71.12) (width 1) (layer "B.Cu") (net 19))
 (segment (start 118.11 49.53) (end 115.57 46.99) (width 1) (layer "B.Cu") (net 19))
 (segment (start 133.35 48.26) (end 137.16 44.45) (width 1) (layer "F.Cu") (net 20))
 (segment (start 130.805 92.715) (end 133.35 90.17) (width 1) (layer "F.Cu") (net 20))
 (segment (start 176.53 71.12) (end 177.8 71.12) (width 1) (layer "F.Cu") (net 20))
 (segment (start 133.35 90.17) (end 133.35 48.26) (width 1) (layer "F.Cu") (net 20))
 (segment (start 175.26 62.23) (end 175.26 69.85) (width 1) (layer "F.Cu") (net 20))
 (segment (start 142.24 44.45) (end 154.94 57.15) (width 1) (layer "F.Cu") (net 20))
 (segment (start 175.26 69.85) (end 176.53 71.12) (width 1) (layer "F.Cu") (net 20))
 (segment (start 154.94 57.15) (end 170.18 57.15) (width 1) (layer "F.Cu") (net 20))
 (segment (start 137.16 44.45) (end 142.24 44.45) (width 1) (layer "F.Cu") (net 20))
 (segment (start 170.18 57.15) (end 175.26 62.23) (width 1) (layer "F.Cu") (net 20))
 (segment (start 125.71 92.715) (end 130.805 92.715) (width 1) (layer "F.Cu") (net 20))
 (segment (start 176.53 71.12) (end 177.8 71.12) (width 1) (layer "B.Cu") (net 20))
 (segment (start 115.57 87.63) (end 120.655 92.715) (width 1) (layer "B.Cu") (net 20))
 (segment (start 177.8 83.82) (end 176.53 83.82) (width 1) (layer "B.Cu") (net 20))
 (segment (start 175.26 82.55) (end 175.26 72.39) (width 1) (layer "B.Cu") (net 20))
 (segment (start 175.26 72.39) (end 176.53 71.12) (width 1) (layer "B.Cu") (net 20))
 (segment (start 115.57 52.07) (end 115.57 87.63) (width 1) (layer "B.Cu") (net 20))
 (segment (start 110.47 49.535) (end 113.035 49.535) (width 1) (layer "B.Cu") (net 20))
 (segment (start 113.035 49.535) (end 115.57 52.07) (width 1) (layer "B.Cu") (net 20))
 (segment (start 176.53 83.82) (end 175.26 82.55) (width 1) (layer "B.Cu") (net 20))
 (segment (start 120.655 92.715) (end 125.71 92.715) (width 1) (layer "B.Cu") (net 20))
 (segment (start 156.21 96.52) (end 149.86 96.52) (width 1) (layer "F.Cu") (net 47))
 (segment (start 147.255 99.125) (end 139.125 99.125) (width 1) (layer "F.Cu") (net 47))
 (segment (start 182.88 88.9) (end 163.83 88.9) (width 1) (layer "F.Cu") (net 47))
 (segment (start 185.42 86.36) (end 182.88 88.9) (width 1) (layer "F.Cu") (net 47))
 (segment (start 185.42 81.28) (end 185.42 86.36) (width 1) (layer "F.Cu") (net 47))
 (segment (start 182.88 78.74) (end 185.42 81.28) (width 1) (layer "F.Cu") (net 47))
 (segment (start 149.86 96.52) (end 147.255 99.125) (width 1) (layer "F.Cu") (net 47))
 (segment (start 163.83 88.9) (end 156.21 96.52) (width 1) (layer "F.Cu") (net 47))
 (segment (start 180.34 78.74) (end 182.88 78.74) (width 1) (layer "F.Cu") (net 47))
 (segment (start 139.125 91.505) (end 142.175 91.505) (width 1) (layer "F.Cu") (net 48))
 (segment (start 162.56 78.74) (end 177.8 78.74) (width 1) (layer "F.Cu") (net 48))
 (segment (start 143.51 91.44) (end 146.05 88.9) (width 1) (layer "F.Cu") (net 48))
 (segment (start 146.05 88.9) (end 152.4 88.9) (width 1) (layer "F.Cu") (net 48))
 (segment (start 142.175 91.505) (end 142.24 91.44) (width 1) (layer "F.Cu") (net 48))
 (segment (start 142.24 91.44) (end 143.51 91.44) (width 1) (layer "F.Cu") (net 48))
 (segment (start 152.4 88.9) (end 162.56 78.74) (width 1) (layer "F.Cu") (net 48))
 (segment (start 153.67 91.44) (end 163.83 81.28) (width 1) (layer "F.Cu") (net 50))
 (segment (start 147.32 91.44) (end 153.67 91.44) (width 1) (layer "F.Cu") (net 50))
 (segment (start 163.83 81.28) (end 177.8 81.28) (width 1) (layer "F.Cu") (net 50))
 (segment (start 139.125 94.045) (end 144.715 94.045) (width 1) (layer "F.Cu") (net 50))
 (segment (start 144.715 94.045) (end 147.32 91.44) (width 1) (layer "F.Cu") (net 50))
 (segment (start 140.905 86.425) (end 143.51 83.82) (width 1) (layer "F.Cu") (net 70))
 (segment (start 143.51 83.82) (end 149.86 83.82) (width 1) (layer "F.Cu") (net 70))
 (segment (start 139.125 86.425) (end 140.905 86.425) (width 1) (layer "F.Cu") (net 70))
 (segment (start 152.4 83.82) (end 152.4 85.09) (width 1) (layer "F.Cu") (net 69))
 (segment (start 142.175 88.965) (end 139.125 88.965) (width 1) (layer "F.Cu") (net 69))
 (segment (start 151.13 86.36) (end 144.78 86.36) (width 1) (layer "F.Cu") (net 69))
 (segment (start 152.4 85.09) (end 151.13 86.36) (width 1) (layer "F.Cu") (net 69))
 (segment (start 144.78 86.36) (end 142.175 88.965) (width 1) (layer "F.Cu") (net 69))
 (segment (start 154.94 93.98) (end 162.56 86.36) (width 1) (layer "F.Cu") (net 49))
 (segment (start 181.61 81.28) (end 180.34 81.28) (width 1) (layer "F.Cu") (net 49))
 (segment (start 182.88 82.55) (end 181.61 81.28) (width 1) (layer "F.Cu") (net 49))
 (segment (start 145.985 96.585) (end 148.59 93.98) (width 1) (layer "F.Cu") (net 49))
 (segment (start 148.59 93.98) (end 154.94 93.98) (width 1) (layer "F.Cu") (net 49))
 (segment (start 181.61 86.36) (end 182.88 85.09) (width 1) (layer "F.Cu") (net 49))
 (segment (start 139.125 96.585) (end 145.985 96.585) (width 1) (layer "F.Cu") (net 49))
 (segment (start 162.56 86.36) (end 181.61 86.36) (width 1) (layer "F.Cu") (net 49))
 (segment (start 182.88 85.09) (end 182.88 82.55) (width 1) (layer "F.Cu") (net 49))
 (segment (start 140.97 101.6) (end 142.24 100.33) (width 1) (layer "B.Cu") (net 28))
 (segment (start 111.765 74.935) (end 113.03 76.2) (width 1) (layer "B.Cu") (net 28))
 (segment (start 142.24 77.47) (end 140.97 76.2) (width 1) (layer "B.Cu") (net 28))
 (segment (start 113.03 88.9) (end 125.73 101.6) (width 1) (layer "B.Cu") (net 28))
 (segment (start 113.03 76.2) (end 113.03 88.9) (width 1) (layer "B.Cu") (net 28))
 (segment (start 140.97 76.2) (end 140.905 76.265) (width 1) (layer "B.Cu") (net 28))
 (segment (start 140.905 76.265) (end 139.125 76.265) (width 1) (layer "B.Cu") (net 28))
 (segment (start 142.24 100.33) (end 142.24 77.47) (width 1) (layer "B.Cu") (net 28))
 (segment (start 125.73 101.6) (end 140.97 101.6) (width 1) (layer "B.Cu") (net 28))
 (segment (start 110.47 74.935) (end 111.765 74.935) (width 1) (layer "B.Cu") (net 28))
 (segment (start 118.105 44.455) (end 118.11 44.45) (width 1) (layer "B.Cu") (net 18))
 (segment (start 95.945 50.865) (end 100.265 50.865) (width 1) (layer "B.Cu") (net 18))
 (segment (start 106.685 44.455) (end 110.47 44.455) (width 1) (layer "B.Cu") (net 18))
 (segment (start 139.125 46.415) (end 139.125 50.865) (width 1) (layer "B.Cu") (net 18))
 (segment (start 128.265 87.635) (end 128.27 87.63) (width 1) (layer "B.Cu") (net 18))
 (segment (start 128.27 46.99) (end 130.81 44.45) (width 1) (layer "B.Cu") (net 18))
 (segment (start 120.65 83.82) (end 124.465 87.635) (width 1) (layer "B.Cu") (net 18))
 (segment (start 130.81 44.45) (end 137.16 44.45) (width 1) (layer "B.Cu") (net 18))
 (segment (start 100.265 50.865) (end 106.68 44.45) (width 1) (layer "B.Cu") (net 18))
 (segment (start 125.71 87.635) (end 128.265 87.635) (width 1) (layer "B.Cu") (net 18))
 (segment (start 120.65 46.99) (end 120.65 83.82) (width 1) (layer "B.Cu") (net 18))
 (segment (start 137.16 44.45) (end 139.125 46.415) (width 1) (layer "B.Cu") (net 18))
 (segment (start 124.465 87.635) (end 125.71 87.635) (width 1) (layer "B.Cu") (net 18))
 (segment (start 128.27 87.63) (end 128.27 46.99) (width 1) (layer "B.Cu") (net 18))
 (segment (start 110.47 44.455) (end 118.105 44.455) (width 1) (layer "B.Cu") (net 18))
 (segment (start 118.11 44.45) (end 120.65 46.99) (width 1) (layer "B.Cu") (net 18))
 (segment (start 106.68 44.45) (end 106.685 44.455) (width 1) (layer "B.Cu") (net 18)))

